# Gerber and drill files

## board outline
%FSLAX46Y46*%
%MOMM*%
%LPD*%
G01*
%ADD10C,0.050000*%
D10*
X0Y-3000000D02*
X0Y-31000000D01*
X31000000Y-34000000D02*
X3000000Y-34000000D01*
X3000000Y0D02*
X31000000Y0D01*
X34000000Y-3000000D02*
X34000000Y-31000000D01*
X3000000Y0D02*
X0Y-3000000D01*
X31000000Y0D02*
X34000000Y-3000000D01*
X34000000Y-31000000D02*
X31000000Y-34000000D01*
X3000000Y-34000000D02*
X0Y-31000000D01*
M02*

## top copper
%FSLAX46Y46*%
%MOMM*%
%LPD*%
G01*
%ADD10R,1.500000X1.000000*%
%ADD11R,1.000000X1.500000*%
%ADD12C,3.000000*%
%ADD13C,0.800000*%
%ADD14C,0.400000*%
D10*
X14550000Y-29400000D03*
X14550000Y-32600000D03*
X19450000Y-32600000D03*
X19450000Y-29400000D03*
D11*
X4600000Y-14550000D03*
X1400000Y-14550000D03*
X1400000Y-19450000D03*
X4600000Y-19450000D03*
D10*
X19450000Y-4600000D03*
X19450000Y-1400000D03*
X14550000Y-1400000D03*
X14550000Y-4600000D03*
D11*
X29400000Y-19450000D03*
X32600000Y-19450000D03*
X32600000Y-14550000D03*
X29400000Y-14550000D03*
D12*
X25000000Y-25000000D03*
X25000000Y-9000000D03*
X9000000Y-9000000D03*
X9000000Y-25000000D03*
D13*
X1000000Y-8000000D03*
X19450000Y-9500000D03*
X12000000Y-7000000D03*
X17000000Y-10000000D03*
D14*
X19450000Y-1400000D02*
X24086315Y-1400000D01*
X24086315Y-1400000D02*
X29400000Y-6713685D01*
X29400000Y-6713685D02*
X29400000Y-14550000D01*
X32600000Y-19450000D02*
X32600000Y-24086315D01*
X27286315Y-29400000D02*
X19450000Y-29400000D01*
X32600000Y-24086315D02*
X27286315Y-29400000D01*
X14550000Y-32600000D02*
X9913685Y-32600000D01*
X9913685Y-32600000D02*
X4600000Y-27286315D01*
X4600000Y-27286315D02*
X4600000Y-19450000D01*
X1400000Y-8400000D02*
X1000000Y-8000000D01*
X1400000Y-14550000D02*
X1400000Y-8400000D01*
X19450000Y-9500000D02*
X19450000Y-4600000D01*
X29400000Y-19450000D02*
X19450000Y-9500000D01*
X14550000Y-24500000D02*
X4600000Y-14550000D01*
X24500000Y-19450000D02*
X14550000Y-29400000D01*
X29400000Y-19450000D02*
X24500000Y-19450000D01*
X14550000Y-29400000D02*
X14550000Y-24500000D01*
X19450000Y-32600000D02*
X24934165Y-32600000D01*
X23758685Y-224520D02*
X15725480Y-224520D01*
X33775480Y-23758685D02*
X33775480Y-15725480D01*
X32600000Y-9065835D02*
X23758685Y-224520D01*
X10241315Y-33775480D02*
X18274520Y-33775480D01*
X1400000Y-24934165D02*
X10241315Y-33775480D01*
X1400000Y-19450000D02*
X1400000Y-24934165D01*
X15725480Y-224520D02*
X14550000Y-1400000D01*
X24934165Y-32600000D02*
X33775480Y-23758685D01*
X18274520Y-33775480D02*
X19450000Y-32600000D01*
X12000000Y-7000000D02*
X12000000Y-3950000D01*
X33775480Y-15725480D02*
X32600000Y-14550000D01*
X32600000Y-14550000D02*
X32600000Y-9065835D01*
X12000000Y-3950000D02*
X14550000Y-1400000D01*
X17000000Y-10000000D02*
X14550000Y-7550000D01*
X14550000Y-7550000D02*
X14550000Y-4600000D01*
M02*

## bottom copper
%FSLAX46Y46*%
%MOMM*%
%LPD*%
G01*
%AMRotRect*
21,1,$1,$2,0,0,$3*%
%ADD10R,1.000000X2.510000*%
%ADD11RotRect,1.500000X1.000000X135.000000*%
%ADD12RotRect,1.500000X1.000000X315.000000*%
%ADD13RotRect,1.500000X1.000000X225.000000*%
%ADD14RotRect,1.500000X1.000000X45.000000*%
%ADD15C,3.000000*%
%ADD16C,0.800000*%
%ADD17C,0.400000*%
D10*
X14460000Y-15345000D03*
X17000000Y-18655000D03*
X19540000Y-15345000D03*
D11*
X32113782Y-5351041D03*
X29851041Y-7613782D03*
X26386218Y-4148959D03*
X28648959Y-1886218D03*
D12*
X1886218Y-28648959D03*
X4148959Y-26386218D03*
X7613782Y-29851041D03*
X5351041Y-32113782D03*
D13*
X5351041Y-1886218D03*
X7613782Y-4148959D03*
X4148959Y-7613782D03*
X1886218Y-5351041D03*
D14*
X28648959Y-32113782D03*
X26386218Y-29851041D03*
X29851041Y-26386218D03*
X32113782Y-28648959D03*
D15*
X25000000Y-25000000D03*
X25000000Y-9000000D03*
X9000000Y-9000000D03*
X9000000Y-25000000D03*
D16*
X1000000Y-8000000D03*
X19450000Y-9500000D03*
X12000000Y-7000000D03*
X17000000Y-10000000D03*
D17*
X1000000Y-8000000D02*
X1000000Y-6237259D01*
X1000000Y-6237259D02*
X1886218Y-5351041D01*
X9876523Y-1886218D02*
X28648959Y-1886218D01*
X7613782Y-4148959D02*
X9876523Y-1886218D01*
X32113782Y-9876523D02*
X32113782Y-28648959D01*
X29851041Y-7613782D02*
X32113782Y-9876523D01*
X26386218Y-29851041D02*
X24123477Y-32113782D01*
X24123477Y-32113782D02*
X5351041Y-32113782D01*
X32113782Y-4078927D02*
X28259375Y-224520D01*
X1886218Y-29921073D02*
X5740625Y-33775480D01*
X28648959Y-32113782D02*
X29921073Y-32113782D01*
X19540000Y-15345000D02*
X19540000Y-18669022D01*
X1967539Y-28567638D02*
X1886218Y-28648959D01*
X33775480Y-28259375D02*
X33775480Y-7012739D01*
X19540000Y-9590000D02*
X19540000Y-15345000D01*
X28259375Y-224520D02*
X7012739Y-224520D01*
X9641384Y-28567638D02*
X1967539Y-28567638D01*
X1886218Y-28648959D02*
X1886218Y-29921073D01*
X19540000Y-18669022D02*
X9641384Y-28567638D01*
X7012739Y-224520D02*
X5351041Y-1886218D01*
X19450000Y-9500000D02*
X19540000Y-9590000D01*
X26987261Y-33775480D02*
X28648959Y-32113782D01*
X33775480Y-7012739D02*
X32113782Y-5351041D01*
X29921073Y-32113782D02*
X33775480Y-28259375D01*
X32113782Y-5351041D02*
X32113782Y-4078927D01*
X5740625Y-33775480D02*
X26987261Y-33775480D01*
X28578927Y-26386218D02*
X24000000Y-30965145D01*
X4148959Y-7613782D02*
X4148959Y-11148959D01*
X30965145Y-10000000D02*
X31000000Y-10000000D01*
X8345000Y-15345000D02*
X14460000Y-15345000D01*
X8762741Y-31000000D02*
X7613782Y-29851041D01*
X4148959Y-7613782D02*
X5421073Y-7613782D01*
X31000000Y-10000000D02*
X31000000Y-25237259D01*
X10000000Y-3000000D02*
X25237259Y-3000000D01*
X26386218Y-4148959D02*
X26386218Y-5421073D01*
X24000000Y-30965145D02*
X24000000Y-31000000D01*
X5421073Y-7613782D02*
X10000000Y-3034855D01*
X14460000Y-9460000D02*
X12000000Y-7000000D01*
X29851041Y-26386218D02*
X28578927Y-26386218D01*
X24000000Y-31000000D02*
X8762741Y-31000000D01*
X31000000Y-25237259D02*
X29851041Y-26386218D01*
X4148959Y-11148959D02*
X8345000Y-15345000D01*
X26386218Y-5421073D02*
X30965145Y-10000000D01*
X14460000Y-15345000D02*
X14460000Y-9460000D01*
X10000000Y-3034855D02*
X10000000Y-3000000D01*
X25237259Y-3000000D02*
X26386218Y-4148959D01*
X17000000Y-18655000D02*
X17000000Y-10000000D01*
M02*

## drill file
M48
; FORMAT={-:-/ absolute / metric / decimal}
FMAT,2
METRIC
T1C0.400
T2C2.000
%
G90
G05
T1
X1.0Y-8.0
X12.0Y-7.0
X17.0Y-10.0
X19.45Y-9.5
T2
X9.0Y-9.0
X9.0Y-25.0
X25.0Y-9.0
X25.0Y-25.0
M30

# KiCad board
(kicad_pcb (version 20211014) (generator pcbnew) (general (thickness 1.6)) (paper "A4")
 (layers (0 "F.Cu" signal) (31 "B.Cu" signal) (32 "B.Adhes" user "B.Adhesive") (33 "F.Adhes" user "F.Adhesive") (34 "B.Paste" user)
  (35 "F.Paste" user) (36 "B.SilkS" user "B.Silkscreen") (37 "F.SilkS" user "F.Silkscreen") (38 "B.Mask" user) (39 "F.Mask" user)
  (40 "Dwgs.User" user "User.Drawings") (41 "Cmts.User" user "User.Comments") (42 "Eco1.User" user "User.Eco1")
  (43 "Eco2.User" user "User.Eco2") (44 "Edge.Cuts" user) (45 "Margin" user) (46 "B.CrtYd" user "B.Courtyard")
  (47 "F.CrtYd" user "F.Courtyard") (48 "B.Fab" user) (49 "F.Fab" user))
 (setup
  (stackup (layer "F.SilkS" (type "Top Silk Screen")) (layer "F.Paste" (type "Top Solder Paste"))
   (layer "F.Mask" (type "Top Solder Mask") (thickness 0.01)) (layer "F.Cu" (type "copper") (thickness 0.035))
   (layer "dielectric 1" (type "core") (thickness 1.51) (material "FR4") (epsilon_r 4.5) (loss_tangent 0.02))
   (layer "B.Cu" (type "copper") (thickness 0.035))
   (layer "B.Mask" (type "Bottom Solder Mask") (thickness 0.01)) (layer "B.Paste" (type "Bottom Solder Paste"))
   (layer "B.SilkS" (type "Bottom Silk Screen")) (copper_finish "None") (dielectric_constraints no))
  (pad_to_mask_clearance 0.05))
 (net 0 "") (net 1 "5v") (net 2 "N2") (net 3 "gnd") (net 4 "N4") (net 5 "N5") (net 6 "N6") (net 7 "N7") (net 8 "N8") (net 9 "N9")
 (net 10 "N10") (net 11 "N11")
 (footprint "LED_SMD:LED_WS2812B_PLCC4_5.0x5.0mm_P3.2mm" (layer "F.Cu") (at 17 31)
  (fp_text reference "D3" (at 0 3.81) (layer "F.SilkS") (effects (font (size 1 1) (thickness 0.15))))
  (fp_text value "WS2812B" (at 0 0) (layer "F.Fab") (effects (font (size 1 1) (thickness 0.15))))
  (pad "1" smd rect locked (at -2.45 -1.6) (size 1.5 1) (layers "F.Cu" "F.Paste" "F.Mask") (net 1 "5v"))
  (pad "2" smd rect locked (at -2.45 1.6) (size 1.5 1) (layers "F.Cu" "F.Paste" "F.Mask") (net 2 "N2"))
  (pad "3" smd rect locked (at 2.45 1.6) (size 1.5 1) (layers "F.Cu" "F.Paste" "F.Mask") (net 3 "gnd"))
  (pad "4" smd rect locked (at 2.45 -1.6) (size 1.5 1) (layers "F.Cu" "F.Paste" "F.Mask") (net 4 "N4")))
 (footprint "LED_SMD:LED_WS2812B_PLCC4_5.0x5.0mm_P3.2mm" (layer "F.Cu") (at 3 17 -90)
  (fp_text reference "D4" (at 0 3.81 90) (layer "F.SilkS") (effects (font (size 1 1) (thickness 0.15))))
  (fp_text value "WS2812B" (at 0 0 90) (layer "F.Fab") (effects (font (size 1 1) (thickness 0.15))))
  (pad "1" smd rect locked (at -2.45 -1.6 270) (size 1.5 1) (layers "F.Cu" "F.Paste" "F.Mask") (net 1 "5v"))
  (pad "2" smd rect locked (at -2.45 1.6 270) (size 1.5 1) (layers "F.Cu" "F.Paste" "F.Mask") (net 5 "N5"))
  (pad "3" smd rect locked (at 2.45 1.6 270) (size 1.5 1) (layers "F.Cu" "F.Paste" "F.Mask") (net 3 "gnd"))
  (pad "4" smd rect locked (at 2.45 -1.6 270) (size 1.5 1) (layers "F.Cu" "F.Paste" "F.Mask") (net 2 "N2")))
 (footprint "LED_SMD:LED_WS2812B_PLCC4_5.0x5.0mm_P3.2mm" (layer "F.Cu") (at 17 3 180)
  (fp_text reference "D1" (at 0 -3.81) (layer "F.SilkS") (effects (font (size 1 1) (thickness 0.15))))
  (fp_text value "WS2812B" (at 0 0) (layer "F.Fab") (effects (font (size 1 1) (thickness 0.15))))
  (pad "1" smd rect locked (at -2.45 -1.6 180) (size 1.5 1) (layers "F.Cu" "F.Paste" "F.Mask") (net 1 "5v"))
  (pad "2" smd rect locked (at -2.45 1.6 180) (size 1.5 1) (layers "F.Cu" "F.Paste" "F.Mask") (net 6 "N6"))
  (pad "3" smd rect locked (at 2.45 1.6 180) (size 1.5 1) (layers "F.Cu" "F.Paste" "F.Mask") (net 3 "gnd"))
  (pad "4" smd rect locked (at 2.45 -1.6 180) (size 1.5 1) (layers "F.Cu" "F.Paste" "F.Mask") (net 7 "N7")))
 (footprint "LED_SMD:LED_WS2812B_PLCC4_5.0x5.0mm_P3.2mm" (layer "F.Cu") (at 31 17 90)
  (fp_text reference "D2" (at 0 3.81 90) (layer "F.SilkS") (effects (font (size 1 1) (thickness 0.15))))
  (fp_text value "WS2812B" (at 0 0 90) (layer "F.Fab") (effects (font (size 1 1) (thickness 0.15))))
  (pad "1" smd rect locked (at -2.45 -1.6 90) (size 1.5 1) (layers "F.Cu" "F.Paste" "F.Mask") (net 1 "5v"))
  (pad "2" smd rect locked (at -2.45 1.6 90) (size 1.5 1) (layers "F.Cu" "F.Paste" "F.Mask") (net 4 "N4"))
  (pad "3" smd rect locked (at 2.45 1.6 90) (size 1.5 1) (layers "F.Cu" "F.Paste" "F.Mask") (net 3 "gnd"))
  (pad "4" smd rect locked (at 2.45 -1.6 90) (size 1.5 1) (layers "F.Cu" "F.Paste" "F.Mask") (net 6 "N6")))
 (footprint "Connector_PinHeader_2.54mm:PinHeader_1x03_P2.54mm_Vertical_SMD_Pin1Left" (layer "B.Cu") (at 17 17 -90)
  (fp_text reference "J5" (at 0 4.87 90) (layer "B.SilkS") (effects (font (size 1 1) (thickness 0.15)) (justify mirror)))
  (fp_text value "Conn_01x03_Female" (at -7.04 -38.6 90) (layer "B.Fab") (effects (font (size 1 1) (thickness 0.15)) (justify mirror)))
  (pad "1" smd rect locked (at -1.655 2.54 270) (size 2.51 1) (layers "B.Cu" "B.Paste" "B.Mask") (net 3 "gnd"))
  (pad "2" smd rect locked (at 1.655 0 270) (size 2.51 1) (layers "B.Cu" "B.Paste" "B.Mask") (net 7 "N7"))
  (pad "3" smd rect locked (at -1.655 -2.54 270) (size 2.51 1) (layers "B.Cu" "B.Paste" "B.Mask") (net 1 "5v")))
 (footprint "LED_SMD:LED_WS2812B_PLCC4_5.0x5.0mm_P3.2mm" (layer "B.Cu") (at 29.25 4.75 135)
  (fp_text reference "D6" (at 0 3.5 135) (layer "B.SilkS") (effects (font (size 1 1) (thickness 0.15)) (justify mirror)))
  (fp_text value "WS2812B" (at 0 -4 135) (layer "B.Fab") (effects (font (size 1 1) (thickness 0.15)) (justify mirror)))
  (pad "1" smd rect (at -2.45 1.6 135) (size 1.5 1) (layers "B.Cu" "B.Paste" "B.Mask") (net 1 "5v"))
  (pad "2" smd rect (at -2.45 -1.6 135) (size 1.5 1) (layers "B.Cu" "B.Paste" "B.Mask") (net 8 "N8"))
  (pad "3" smd rect (at 2.45 -1.6 135) (size 1.5 1) (layers "B.Cu" "B.Paste" "B.Mask") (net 3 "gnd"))
  (pad "4" smd rect (at 2.45 1.6 135) (size 1.5 1) (layers "B.Cu" "B.Paste" "B.Mask") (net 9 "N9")))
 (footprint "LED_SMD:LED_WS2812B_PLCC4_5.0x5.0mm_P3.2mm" (layer "B.Cu") (at 4.75 29.25 -45)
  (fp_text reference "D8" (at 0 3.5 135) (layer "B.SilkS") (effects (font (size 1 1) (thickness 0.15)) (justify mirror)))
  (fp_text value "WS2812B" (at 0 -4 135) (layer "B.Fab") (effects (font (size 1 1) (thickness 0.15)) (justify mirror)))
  (pad "1" smd rect (at -2.45 1.6 315) (size 1.5 1) (layers "B.Cu" "B.Paste" "B.Mask") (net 1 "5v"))
  (pad "2" smd rect (at -2.45 -1.6 315) (size 1.5 1) (layers "B.Cu" "B.Paste" "B.Mask") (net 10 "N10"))
  (pad "3" smd rect (at 2.45 -1.6 315) (size 1.5 1) (layers "B.Cu" "B.Paste" "B.Mask") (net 3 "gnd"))
  (pad "4" smd rect (at 2.45 1.6 315) (size 1.5 1) (layers "B.Cu" "B.Paste" "B.Mask") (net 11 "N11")))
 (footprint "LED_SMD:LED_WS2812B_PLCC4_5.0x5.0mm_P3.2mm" (layer "B.Cu") (at 4.75 4.75 -135)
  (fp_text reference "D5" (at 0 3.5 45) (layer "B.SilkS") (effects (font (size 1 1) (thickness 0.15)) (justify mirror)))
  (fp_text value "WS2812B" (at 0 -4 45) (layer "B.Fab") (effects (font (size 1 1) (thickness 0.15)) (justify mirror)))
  (pad "1" smd rect (at -2.45 1.6 225) (size 1.5 1) (layers "B.Cu" "B.Paste" "B.Mask") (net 1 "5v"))
  (pad "2" smd rect (at -2.45 -1.6 225) (size 1.5 1) (layers "B.Cu" "B.Paste" "B.Mask") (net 9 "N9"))
  (pad "3" smd rect (at 2.45 -1.6 225) (size 1.5 1) (layers "B.Cu" "B.Paste" "B.Mask") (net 3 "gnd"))
  (pad "4" smd rect (at 2.45 1.6 225) (size 1.5 1) (layers "B.Cu" "B.Paste" "B.Mask") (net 5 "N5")))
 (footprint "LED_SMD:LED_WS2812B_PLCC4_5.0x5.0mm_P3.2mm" (layer "B.Cu") (at 29.25 29.25 45)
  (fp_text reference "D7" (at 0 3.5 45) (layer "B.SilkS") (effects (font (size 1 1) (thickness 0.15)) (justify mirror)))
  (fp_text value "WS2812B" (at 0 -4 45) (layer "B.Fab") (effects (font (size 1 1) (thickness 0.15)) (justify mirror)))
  (pad "1" smd rect (at -2.45 1.6 45) (size 1.5 1) (layers "B.Cu" "B.Paste" "B.Mask") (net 1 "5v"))
  (pad "2" smd rect (at -2.45 -1.6 45) (size 1.5 1) (layers "B.Cu" "B.Paste" "B.Mask") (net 11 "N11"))
  (pad "3" smd rect (at 2.45 -1.6 45) (size 1.5 1) (layers "B.Cu" "B.Paste" "B.Mask") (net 3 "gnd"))
  (pad "4" smd rect (at 2.45 1.6 45) (size 1.5 1) (layers "B.Cu" "B.Paste" "B.Mask") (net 8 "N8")))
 (gr_line (start 0 3) (end 0 31) (layer "Edge.Cuts") (width 0.05))
 (gr_line (start 31 34) (end 3 34) (layer "Edge.Cuts") (width 0.05))
 (gr_line (start 3 0) (end 31 0) (layer "Edge.Cuts") (width 0.05))
 (gr_line (start 34 3) (end 34 31) (layer "Edge.Cuts") (width 0.05))
 (gr_line (start 3 0) (end 0 3) (layer "Edge.Cuts") (width 0.05))
 (gr_line (start 31 0) (end 34 3) (layer "Edge.Cuts") (width 0.05))
 (gr_line (start 34 31) (end 31 34) (layer "Edge.Cuts") (width 0.05))
 (gr_line (start 3 34) (end 0 31) (layer "Edge.Cuts") (width 0.05))
 (via (at 25 25) (size 3) (drill 2) (layers "F.Cu" "B.Cu") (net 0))
 (via (at 25 9) (size 3) (drill 2) (layers "F.Cu" "B.Cu") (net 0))
 (via (at 9 9) (size 3) (drill 2) (layers "F.Cu" "B.Cu") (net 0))
 (via (at 9 25) (size 3) (drill 2) (layers "F.Cu" "B.Cu") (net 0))
 (segment (start 19.45 1.4) (end 24.086315 1.4) (width 0.4) (layer "F.Cu") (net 6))
 (segment (start 24.086315 1.4) (end 29.4 6.713685) (width 0.4) (layer "F.Cu") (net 6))
 (segment (start 29.4 6.713685) (end 29.4 14.55) (width 0.4) (layer "F.Cu") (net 6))
 (segment (start 32.6 19.45) (end 32.6 24.086315) (width 0.4) (layer "F.Cu") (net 4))
 (segment (start 27.286315 29.4) (end 19.45 29.4) (width 0.4) (layer "F.Cu") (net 4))
 (segment (start 32.6 24.086315) (end 27.286315 29.4) (width 0.4) (layer "F.Cu") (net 4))
 (segment (start 14.55 32.6) (end 9.913685 32.6) (width 0.4) (layer "F.Cu") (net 2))
 (segment (start 9.913685 32.6) (end 4.6 27.286315) (width 0.4) (layer "F.Cu") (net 2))
 (segment (start 4.6 27.286315) (end 4.6 19.45) (width 0.4) (layer "F.Cu") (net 2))
 (segment (start 1.4 8.4) (end 1 8) (width 0.4) (layer "F.Cu") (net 5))
 (segment (start 1.4 14.55) (end 1.4 8.4) (width 0.4) (layer "F.Cu") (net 5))
 (via (at 1 8) (size 0.8) (drill 0.4) (layers "F.Cu" "B.Cu") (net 5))
 (segment (start 1 8) (end 1 6.237259) (width 0.4) (layer "B.Cu") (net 5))
 (segment (start 1 6.237259) (end 1.886218 5.351041) (width 0.4) (layer "B.Cu") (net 5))
 (segment (start 9.876523 1.886218) (end 28.648959 1.886218) (width 0.4) (layer "B.Cu") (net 9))
 (segment (start 7.613782 4.148959) (end 9.876523 1.886218) (width 0.4) (layer "B.Cu") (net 9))
 (segment (start 32.113782 9.876523) (end 32.113782 28.648959) (width 0.4) (layer "B.Cu") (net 8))
 (segment (start 29.851041 7.613782) (end 32.113782 9.876523) (width 0.4) (layer "B.Cu") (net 8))
 (segment (start 26.386218 29.851041) (end 24.123477 32.113782) (width 0.4) (layer "B.Cu") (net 11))
 (segment (start 24.123477 32.113782) (end 5.351041 32.113782) (width 0.4) (layer "B.Cu") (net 11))
 (segment (start 19.45 9.5) (end 19.45 4.6) (width 0.4) (layer "F.Cu") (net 1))
 (segment (start 29.4 19.45) (end 19.45 9.5) (width 0.4) (layer "F.Cu") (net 1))
 (segment (start 14.55 24.5) (end 4.6 14.55) (width 0.4) (layer "F.Cu") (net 1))
 (segment (start 24.5 19.45) (end 14.55 29.4) (width 0.4) (layer "F.Cu") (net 1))
 (segment (start 29.4 19.45) (end 24.5 19.45) (width 0.4) (layer "F.Cu") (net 1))
 (segment (start 14.55 29.4) (end 14.55 24.5) (width 0.4) (layer "F.Cu") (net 1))
 (via (at 19.45 9.5) (size 0.8) (drill 0.4) (layers "F.Cu" "B.Cu") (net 1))
 (segment (start 32.113782 4.078927) (end 28.259375 0.22452) (width 0.4) (layer "B.Cu") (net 1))
 (segment (start 1.886218 29.921073) (end 5.740625 33.77548) (width 0.4) (layer "B.Cu") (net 1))
 (segment (start 28.648959 32.113782) (end 29.921073 32.113782) (width 0.4) (layer "B.Cu") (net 1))
 (segment (start 19.54 15.345) (end 19.54 18.669022) (width 0.4) (layer "B.Cu") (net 1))
 (segment (start 1.967539 28.567638) (end 1.886218 28.648959) (width 0.4) (layer "B.Cu") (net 1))
 (segment (start 33.77548 28.259375) (end 33.77548 7.012739) (width 0.4) (layer "B.Cu") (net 1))
 (segment (start 19.54 9.59) (end 19.54 15.345) (width 0.4) (layer "B.Cu") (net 1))
 (segment (start 28.259375 0.22452) (end 7.012739 0.22452) (width 0.4) (layer "B.Cu") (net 1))
 (segment (start 9.641384 28.567638) (end 1.967539 28.567638) (width 0.4) (layer "B.Cu") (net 1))
 (segment (start 1.886218 28.648959) (end 1.886218 29.921073) (width 0.4) (layer "B.Cu") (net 1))
 (segment (start 19.54 18.669022) (end 9.641384 28.567638) (width 0.4) (layer "B.Cu") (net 1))
 (segment (start 7.012739 0.22452) (end 5.351041 1.886218) (width 0.4) (layer "B.Cu") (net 1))
 (segment (start 19.45 9.5) (end 19.54 9.59) (width 0.4) (layer "B.Cu") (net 1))
 (segment (start 26.987261 33.77548) (end 28.648959 32.113782) (width 0.4) (layer "B.Cu") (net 1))
 (segment (start 33.77548 7.012739) (end 32.113782 5.351041) (width 0.4) (layer "B.Cu") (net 1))
 (segment (start 29.921073 32.113782) (end 33.77548 28.259375) (width 0.4) (layer "B.Cu") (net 1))
 (segment (start 32.113782 5.351041) (end 32.113782 4.078927) (width 0.4) (layer "B.Cu") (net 1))
 (segment (start 5.740625 33.77548) (end 26.987261 33.77548) (width 0.4) (layer "B.Cu") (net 1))
 (segment (start 19.45 32.6) (end 24.934165 32.6) (width 0.4) (layer "F.Cu") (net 3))
 (segment (start 23.758685 0.22452) (end 15.72548 0.22452) (width 0.4) (layer "F.Cu") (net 3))
 (segment (start 33.77548 23.758685) (end 33.77548 15.72548) (width 0.4) (layer "F.Cu") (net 3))
 (segment (start 32.6 9.065835) (end 23.758685 0.22452) (width 0.4) (layer "F.Cu") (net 3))
 (segment (start 10.241315 33.77548) (end 18.27452 33.77548) (width 0.4) (layer "F.Cu") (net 3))
 (segment (start 1.4 24.934165) (end 10.241315 33.77548) (width 0.4) (layer "F.Cu") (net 3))
 (segment (start 1.4 19.45) (end 1.4 24.934165) (width 0.4) (layer "F.Cu") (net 3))
 (segment (start 15.72548 0.22452) (end 14.55 1.4) (width 0.4) (layer "F.Cu") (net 3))
 (segment (start 24.934165 32.6) (end 33.77548 23.758685) (width 0.4) (layer "F.Cu") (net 3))
 (segment (start 18.27452 33.77548) (end 19.45 32.6) (width 0.4) (layer "F.Cu") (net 3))
 (segment (start 12 7) (end 12 3.95) (width 0.4) (layer "F.Cu") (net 3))
 (segment (start 33.77548 15.72548) (end 32.6 14.55) (width 0.4) (layer "F.Cu") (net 3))
 (segment (start 32.6 14.55) (end 32.6 9.065835) (width 0.4) (layer "F.Cu") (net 3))
 (segment (start 12 3.95) (end 14.55 1.4) (width 0.4) (layer "F.Cu") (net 3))
 (via (at 12 7) (size 0.8) (drill 0.4) (layers "F.Cu" "B.Cu") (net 3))
 (segment (start 28.578927 26.386218) (end 24 30.965145) (width 0.4) (layer "B.Cu") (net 3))
 (segment (start 4.148959 7.613782) (end 4.148959 11.148959) (width 0.4) (layer "B.Cu") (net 3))
 (segment (start 30.965145 10) (end 31 10) (width 0.4) (layer "B.Cu") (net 3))
 (segment (start 8.345 15.345) (end 14.46 15.345) (width 0.4) (layer "B.Cu") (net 3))
 (segment (start 8.762741 31) (end 7.613782 29.851041) (width 0.4) (layer "B.Cu") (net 3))
 (segment (start 4.148959 7.613782) (end 5.421073 7.613782) (width 0.4) (layer "B.Cu") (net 3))
 (segment (start 31 10) (end 31 25.237259) (width 0.4) (layer "B.Cu") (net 3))
 (segment (start 10 3) (end 25.237259 3) (width 0.4) (layer "B.Cu") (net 3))
 (segment (start 26.386218 4.148959) (end 26.386218 5.421073) (width 0.4) (layer "B.Cu") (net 3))
 (segment (start 24 30.965145) (end 24 31) (width 0.4) (layer "B.Cu") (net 3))
 (segment (start 5.421073 7.613782) (end 10 3.034855) (width 0.4) (layer "B.Cu") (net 3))
 (segment (start 14.46 9.46) (end 12 7) (width 0.4) (layer "B.Cu") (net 3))
 (segment (start 29.851041 26.386218) (end 28.578927 26.386218) (width 0.4) (layer "B.Cu") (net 3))
 (segment (start 24 31) (end 8.762741 31) (width 0.4) (layer "B.Cu") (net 3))
 (segment (start 31 25.237259) (end 29.851041 26.386218) (width 0.4) (layer "B.Cu") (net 3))
 (segment (start 4.148959 11.148959) (end 8.345 15.345) (width 0.4) (layer "B.Cu") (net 3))
 (segment (start 26.386218 5.421073) (end 30.965145 10) (width 0.4) (layer "B.Cu") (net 3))
 (segment (start 14.46 15.345) (end 14.46 9.46) (width 0.4) (layer "B.Cu") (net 3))
 (segment (start 10 3.034855) (end 10 3) (width 0.4) (layer "B.Cu") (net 3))
 (segment (start 25.237259 3) (end 26.386218 4.148959) (width 0.4) (layer "B.Cu") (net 3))
 (segment (start 17 10) (end 14.55 7.55) (width 0.4) (layer "F.Cu") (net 7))
 (segment (start 14.55 7.55) (end 14.55 4.6) (width 0.4) (layer "F.Cu") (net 7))
 (via (at 17 10) (size 0.8) (drill 0.4) (layers "F.Cu" "B.Cu") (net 7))
 (segment (start 17 18.655) (end 17 10) (width 0.4) (layer "B.Cu") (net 7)))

